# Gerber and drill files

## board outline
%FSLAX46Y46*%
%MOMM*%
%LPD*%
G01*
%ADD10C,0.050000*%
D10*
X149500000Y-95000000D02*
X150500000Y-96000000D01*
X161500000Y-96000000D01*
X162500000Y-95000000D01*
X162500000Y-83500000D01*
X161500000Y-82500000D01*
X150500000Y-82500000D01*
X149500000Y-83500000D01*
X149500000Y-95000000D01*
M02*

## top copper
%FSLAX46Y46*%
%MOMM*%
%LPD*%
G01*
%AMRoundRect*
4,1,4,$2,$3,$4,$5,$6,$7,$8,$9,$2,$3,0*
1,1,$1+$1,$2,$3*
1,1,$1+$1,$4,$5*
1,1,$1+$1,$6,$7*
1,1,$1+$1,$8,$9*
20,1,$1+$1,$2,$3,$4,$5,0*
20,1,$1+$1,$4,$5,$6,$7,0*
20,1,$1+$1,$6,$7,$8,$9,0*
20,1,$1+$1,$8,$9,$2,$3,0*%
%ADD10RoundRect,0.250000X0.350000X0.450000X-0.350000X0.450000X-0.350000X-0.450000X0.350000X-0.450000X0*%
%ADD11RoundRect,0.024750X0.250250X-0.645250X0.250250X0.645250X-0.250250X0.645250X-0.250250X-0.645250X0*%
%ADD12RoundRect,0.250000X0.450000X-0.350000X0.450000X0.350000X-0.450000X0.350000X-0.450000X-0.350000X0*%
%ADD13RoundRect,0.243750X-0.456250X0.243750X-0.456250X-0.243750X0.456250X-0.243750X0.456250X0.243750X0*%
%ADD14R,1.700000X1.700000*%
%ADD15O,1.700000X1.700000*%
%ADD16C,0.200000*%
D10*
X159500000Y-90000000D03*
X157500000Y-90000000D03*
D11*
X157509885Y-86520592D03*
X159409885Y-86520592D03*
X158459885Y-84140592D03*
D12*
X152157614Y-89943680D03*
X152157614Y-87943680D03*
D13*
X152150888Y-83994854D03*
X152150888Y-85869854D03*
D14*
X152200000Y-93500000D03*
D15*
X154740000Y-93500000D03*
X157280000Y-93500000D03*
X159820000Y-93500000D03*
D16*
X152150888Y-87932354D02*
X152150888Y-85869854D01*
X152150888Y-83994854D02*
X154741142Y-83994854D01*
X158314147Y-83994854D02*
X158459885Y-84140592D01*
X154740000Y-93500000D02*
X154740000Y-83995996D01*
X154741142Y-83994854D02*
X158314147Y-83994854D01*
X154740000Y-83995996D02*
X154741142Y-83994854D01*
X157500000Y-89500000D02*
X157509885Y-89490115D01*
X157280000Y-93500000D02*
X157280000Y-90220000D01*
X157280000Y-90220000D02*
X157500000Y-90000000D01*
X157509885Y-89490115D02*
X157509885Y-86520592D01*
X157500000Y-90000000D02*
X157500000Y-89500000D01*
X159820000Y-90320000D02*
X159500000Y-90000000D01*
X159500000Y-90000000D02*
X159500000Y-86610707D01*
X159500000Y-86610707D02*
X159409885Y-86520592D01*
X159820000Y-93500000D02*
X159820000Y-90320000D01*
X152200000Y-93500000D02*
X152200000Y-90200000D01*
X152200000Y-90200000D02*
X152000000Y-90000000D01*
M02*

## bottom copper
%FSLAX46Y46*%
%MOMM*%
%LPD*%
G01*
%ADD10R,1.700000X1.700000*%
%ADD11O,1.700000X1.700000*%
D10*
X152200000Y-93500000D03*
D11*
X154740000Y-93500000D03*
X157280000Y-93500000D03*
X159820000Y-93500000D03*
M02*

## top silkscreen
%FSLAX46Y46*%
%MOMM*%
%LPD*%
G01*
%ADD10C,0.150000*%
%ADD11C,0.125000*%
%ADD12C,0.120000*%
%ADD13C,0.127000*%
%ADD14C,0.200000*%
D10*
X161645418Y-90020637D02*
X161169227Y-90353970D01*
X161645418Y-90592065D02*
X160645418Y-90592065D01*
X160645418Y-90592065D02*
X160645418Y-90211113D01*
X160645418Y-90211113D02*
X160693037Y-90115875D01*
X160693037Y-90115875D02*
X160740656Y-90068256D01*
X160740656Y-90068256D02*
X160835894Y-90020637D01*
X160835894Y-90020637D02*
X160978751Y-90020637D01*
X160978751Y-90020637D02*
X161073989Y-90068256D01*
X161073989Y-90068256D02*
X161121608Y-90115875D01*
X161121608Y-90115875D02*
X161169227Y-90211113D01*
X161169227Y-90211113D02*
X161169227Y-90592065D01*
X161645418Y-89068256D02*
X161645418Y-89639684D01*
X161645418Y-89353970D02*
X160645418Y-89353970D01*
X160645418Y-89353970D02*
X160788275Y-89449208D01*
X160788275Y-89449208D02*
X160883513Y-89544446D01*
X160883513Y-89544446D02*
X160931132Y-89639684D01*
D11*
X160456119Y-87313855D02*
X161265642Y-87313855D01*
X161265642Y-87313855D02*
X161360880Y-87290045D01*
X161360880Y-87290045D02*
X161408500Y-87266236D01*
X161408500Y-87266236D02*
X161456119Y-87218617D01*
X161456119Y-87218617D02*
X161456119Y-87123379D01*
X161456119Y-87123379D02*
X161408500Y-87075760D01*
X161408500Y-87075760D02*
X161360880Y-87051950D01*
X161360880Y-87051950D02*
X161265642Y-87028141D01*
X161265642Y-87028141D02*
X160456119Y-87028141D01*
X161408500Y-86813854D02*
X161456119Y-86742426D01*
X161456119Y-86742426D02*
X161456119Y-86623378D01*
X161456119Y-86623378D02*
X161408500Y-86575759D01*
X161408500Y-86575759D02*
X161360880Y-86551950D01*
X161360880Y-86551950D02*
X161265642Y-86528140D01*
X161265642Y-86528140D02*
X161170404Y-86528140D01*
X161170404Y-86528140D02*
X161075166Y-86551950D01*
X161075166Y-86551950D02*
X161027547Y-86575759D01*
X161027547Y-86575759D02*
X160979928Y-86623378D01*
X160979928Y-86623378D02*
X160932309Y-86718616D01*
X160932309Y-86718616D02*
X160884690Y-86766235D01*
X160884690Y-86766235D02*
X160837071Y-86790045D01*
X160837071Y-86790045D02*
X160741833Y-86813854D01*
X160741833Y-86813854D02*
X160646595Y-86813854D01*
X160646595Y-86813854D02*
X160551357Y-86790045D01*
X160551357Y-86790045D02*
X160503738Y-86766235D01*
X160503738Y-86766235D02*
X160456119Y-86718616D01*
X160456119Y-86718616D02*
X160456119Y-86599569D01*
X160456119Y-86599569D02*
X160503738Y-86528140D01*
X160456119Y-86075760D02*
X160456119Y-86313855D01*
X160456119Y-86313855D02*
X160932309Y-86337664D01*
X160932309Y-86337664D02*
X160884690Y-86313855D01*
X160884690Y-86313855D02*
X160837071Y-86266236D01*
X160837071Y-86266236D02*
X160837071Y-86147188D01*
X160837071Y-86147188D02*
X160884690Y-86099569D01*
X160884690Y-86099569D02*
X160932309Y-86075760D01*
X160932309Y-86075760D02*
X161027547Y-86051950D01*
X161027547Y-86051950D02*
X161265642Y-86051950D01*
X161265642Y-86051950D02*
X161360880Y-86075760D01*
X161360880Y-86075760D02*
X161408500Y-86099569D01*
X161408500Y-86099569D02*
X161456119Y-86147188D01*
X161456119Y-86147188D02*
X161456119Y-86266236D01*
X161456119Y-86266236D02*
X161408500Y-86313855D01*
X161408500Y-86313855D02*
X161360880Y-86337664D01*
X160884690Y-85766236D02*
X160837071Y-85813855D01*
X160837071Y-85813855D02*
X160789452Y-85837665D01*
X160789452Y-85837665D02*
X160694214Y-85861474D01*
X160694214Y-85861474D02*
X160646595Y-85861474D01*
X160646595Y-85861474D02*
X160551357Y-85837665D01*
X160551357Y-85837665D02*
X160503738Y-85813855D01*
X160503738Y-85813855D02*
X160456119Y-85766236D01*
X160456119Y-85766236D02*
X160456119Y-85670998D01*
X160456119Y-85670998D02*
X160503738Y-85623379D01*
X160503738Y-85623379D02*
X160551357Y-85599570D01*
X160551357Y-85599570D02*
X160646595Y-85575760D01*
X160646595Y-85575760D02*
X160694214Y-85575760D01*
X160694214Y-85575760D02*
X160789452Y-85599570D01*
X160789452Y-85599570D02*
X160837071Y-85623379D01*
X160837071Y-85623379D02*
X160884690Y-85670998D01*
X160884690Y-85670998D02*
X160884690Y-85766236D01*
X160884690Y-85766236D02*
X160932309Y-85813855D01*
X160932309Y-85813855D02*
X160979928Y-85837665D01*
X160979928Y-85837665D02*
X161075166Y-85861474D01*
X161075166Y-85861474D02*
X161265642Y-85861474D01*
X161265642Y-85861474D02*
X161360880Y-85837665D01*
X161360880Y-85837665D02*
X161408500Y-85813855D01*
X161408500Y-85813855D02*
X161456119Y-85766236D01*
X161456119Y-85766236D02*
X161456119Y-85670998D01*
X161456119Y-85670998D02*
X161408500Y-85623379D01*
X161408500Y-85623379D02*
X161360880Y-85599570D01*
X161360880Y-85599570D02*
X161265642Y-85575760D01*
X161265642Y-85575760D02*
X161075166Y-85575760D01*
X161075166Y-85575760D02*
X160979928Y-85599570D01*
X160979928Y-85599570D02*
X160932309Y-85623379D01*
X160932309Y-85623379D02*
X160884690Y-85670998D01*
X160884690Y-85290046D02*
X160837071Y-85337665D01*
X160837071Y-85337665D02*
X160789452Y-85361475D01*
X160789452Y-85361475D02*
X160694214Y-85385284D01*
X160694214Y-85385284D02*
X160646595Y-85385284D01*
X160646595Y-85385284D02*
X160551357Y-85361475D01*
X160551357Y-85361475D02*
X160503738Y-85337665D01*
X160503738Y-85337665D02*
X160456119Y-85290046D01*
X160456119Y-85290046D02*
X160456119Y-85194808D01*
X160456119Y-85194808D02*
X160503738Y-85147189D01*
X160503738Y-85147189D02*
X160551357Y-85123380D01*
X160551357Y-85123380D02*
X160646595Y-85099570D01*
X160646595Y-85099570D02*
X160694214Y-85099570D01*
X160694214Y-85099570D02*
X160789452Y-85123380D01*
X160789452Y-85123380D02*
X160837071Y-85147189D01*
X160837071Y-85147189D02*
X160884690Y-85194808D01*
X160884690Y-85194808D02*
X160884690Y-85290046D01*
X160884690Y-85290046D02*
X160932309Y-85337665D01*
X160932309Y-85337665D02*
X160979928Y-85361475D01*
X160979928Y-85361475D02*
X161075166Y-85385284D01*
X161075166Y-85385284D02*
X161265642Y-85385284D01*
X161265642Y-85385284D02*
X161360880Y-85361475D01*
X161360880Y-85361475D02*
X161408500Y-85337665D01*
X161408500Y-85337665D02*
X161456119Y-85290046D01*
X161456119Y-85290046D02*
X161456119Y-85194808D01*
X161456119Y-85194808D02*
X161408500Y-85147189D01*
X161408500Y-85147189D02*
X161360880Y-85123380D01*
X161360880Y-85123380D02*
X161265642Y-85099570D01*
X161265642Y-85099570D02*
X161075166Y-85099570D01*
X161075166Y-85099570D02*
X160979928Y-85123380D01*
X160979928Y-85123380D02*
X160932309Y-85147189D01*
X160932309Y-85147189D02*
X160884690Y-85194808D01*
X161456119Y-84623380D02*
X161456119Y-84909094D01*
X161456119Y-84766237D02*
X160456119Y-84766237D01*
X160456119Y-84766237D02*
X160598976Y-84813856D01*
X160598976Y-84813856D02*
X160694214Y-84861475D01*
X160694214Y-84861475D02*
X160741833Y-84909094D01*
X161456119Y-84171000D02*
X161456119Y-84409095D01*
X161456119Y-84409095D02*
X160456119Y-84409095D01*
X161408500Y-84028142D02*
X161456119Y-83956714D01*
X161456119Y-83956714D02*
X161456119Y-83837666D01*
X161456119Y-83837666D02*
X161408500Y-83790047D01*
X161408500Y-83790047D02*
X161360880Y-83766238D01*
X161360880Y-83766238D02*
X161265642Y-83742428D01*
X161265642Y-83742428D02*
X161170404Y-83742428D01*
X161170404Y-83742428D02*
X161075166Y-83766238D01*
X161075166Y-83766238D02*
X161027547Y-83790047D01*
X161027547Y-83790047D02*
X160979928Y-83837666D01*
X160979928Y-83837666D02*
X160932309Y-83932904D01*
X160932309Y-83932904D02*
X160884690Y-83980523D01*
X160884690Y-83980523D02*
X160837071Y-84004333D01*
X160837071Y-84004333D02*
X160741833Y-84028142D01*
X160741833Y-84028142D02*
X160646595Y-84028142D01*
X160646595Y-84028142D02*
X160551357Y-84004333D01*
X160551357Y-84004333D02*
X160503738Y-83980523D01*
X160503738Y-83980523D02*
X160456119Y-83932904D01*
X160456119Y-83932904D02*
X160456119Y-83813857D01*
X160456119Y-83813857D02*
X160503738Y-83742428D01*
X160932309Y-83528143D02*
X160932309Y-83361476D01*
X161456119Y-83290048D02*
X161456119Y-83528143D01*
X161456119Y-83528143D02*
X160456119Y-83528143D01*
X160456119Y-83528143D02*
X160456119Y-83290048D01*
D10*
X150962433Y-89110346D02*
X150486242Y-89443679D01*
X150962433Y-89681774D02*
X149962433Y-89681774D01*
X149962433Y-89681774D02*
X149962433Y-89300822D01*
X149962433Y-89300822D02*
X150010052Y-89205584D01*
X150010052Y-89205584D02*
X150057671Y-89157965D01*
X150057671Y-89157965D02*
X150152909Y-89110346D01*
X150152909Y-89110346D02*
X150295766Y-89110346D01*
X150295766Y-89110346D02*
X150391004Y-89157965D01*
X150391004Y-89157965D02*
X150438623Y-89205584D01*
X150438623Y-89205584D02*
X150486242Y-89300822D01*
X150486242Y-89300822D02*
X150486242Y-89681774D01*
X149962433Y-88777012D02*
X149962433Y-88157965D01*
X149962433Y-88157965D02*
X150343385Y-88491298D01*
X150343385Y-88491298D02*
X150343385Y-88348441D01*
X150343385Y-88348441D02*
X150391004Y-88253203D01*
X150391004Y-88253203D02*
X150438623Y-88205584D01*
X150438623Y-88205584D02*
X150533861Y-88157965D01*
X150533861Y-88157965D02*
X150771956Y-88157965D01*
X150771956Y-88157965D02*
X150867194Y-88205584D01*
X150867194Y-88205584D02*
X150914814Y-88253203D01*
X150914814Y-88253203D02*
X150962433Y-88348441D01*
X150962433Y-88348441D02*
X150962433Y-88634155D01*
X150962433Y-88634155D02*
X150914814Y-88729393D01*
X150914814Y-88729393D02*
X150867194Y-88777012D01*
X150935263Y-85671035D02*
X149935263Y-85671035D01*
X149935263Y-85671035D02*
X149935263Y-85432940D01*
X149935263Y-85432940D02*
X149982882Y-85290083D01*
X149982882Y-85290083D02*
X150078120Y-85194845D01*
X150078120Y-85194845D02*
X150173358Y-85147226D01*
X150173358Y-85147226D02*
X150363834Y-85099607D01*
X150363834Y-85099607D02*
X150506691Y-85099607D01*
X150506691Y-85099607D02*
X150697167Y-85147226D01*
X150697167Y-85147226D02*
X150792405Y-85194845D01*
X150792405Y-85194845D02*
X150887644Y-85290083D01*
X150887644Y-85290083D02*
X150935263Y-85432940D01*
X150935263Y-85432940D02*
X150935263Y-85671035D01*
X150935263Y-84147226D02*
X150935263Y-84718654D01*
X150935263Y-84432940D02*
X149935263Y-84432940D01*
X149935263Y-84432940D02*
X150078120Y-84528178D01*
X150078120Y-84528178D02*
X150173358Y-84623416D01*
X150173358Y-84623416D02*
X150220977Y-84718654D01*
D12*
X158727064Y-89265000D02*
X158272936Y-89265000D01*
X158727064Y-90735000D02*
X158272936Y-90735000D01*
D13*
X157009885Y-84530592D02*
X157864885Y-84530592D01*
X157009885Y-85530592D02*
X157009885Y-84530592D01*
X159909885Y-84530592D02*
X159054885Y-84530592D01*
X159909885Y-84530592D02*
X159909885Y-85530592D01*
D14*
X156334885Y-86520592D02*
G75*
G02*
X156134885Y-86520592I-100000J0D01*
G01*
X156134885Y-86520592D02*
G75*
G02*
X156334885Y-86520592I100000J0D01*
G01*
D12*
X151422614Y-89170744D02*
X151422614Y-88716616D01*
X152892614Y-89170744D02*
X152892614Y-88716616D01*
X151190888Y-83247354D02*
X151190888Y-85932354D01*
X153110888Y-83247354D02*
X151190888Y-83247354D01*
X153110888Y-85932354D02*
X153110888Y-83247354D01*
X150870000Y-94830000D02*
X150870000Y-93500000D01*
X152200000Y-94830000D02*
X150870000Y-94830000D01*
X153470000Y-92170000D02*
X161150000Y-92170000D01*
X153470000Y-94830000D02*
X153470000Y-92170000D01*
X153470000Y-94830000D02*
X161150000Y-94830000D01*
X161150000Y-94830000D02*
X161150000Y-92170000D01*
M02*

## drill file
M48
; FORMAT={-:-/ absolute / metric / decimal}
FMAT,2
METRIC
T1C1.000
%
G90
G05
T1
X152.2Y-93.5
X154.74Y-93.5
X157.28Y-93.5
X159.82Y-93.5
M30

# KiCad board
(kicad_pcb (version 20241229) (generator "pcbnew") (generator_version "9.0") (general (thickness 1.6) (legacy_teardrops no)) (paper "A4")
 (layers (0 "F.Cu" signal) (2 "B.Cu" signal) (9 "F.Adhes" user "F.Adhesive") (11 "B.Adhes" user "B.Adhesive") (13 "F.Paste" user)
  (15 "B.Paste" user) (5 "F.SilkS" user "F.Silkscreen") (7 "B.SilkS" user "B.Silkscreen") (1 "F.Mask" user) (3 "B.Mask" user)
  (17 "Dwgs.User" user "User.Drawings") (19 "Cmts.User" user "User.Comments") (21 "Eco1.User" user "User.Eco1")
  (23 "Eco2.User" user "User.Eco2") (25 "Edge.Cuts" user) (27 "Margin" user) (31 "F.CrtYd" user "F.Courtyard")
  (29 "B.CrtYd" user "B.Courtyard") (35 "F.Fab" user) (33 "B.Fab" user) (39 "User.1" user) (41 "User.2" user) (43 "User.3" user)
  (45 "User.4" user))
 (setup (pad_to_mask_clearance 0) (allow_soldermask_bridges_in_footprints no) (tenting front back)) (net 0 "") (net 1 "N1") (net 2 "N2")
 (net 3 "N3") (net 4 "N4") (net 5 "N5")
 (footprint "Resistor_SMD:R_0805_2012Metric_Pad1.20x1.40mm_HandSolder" (layer "F.Cu") (at 158.5 90 180)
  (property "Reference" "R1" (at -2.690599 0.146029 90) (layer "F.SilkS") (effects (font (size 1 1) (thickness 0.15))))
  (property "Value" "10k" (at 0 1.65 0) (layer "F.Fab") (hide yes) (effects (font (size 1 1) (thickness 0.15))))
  (fp_line (start -0.227064 0.735) (end 0.227064 0.735) (stroke (width 0.12) (type solid)) (layer "F.SilkS"))
  (fp_line (start -0.227064 -0.735) (end 0.227064 -0.735) (stroke (width 0.12) (type solid)) (layer "F.SilkS"))
  (pad "1" smd roundrect (at -1 0 180) (size 1.2 1.4) (layers "F.Cu" "F.Mask" "F.Paste") (roundrect_rratio 0.208333) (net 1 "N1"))
  (pad "2" smd roundrect (at 1 0 180) (size 1.2 1.4) (layers "F.Cu" "F.Mask" "F.Paste") (roundrect_rratio 0.208333) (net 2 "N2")))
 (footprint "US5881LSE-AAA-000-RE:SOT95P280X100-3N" (layer "F.Cu") (at 158.459885 85.330592 90)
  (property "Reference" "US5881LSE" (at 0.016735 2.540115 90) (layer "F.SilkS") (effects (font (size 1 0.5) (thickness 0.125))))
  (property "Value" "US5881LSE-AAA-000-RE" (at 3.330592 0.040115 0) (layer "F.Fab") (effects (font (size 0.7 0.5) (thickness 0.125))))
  (fp_line (start 0.8 -1.45) (end 0.8 -0.595) (stroke (width 0.127) (type solid)) (layer "F.SilkS"))
  (fp_line (start -0.2 -1.45) (end 0.8 -1.45) (stroke (width 0.127) (type solid)) (layer "F.SilkS"))
  (fp_line (start 0.8 1.45) (end 0.8 0.595) (stroke (width 0.127) (type solid)) (layer "F.SilkS"))
  (fp_line (start 0.8 1.45) (end -0.2 1.45) (stroke (width 0.127) (type solid)) (layer "F.SilkS"))
  (fp_circle (center -1.19 -2.225) (end -1.09 -2.225) (stroke (width 0.2) (type solid)) (fill no) (layer "F.SilkS"))
  (pad "1" smd roundrect (at -1.19 -0.95 90) (size 1.34 0.55) (layers "F.Cu" "F.Mask" "F.Paste") (roundrect_rratio 0.045) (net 2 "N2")
   (solder_mask_margin 0.102))
  (pad "2" smd roundrect (at -1.19 0.95 90) (size 1.34 0.55) (layers "F.Cu" "F.Mask" "F.Paste") (roundrect_rratio 0.045) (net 1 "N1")
   (solder_mask_margin 0.102))
  (pad "3" smd roundrect (at 1.19 0 90) (size 1.34 0.55) (layers "F.Cu" "F.Mask" "F.Paste") (roundrect_rratio 0.045) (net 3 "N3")
   (solder_mask_margin 0.102)))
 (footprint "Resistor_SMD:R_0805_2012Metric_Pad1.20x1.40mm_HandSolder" (layer "F.Cu") (at 152.157614 88.94368 90)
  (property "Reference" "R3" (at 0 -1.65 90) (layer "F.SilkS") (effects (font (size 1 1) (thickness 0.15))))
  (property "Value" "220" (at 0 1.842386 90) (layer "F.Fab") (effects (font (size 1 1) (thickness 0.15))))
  (fp_line (start -0.227064 -0.735) (end 0.227064 -0.735) (stroke (width 0.12) (type solid)) (layer "F.SilkS"))
  (fp_line (start -0.227064 0.735) (end 0.227064 0.735) (stroke (width 0.12) (type solid)) (layer "F.SilkS"))
  (pad "1" smd roundrect (at -1 0 90) (size 1.2 1.4) (layers "F.Cu" "F.Mask" "F.Paste") (roundrect_rratio 0.208333) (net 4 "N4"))
  (pad "2" smd roundrect (at 1 0 90) (size 1.2 1.4) (layers "F.Cu" "F.Mask" "F.Paste") (roundrect_rratio 0.208333) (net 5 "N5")))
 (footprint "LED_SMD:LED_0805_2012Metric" (layer "F.Cu") (at 152.150888 84.932354 -90)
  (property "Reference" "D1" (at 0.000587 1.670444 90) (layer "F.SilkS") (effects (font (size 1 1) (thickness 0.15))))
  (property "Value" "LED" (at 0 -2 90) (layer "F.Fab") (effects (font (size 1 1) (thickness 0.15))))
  (fp_line (start -1.685 0.96) (end 1 0.96) (stroke (width 0.12) (type solid)) (layer "F.SilkS"))
  (fp_line (start -1.685 -0.96) (end -1.685 0.96) (stroke (width 0.12) (type solid)) (layer "F.SilkS"))
  (fp_line (start 1 -0.96) (end -1.685 -0.96) (stroke (width 0.12) (type solid)) (layer "F.SilkS"))
  (pad "1" smd roundrect (at -0.9375 0 270) (size 0.975 1.4) (layers "F.Cu" "F.Mask" "F.Paste") (roundrect_rratio 0.25) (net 3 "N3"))
  (pad "2" smd roundrect (at 0.9375 0 270) (size 0.975 1.4) (layers "F.Cu" "F.Mask" "F.Paste") (roundrect_rratio 0.25) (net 5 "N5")))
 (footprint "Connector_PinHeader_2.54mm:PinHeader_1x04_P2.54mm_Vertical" (layer "F.Cu") (at 152.2 93.5 90)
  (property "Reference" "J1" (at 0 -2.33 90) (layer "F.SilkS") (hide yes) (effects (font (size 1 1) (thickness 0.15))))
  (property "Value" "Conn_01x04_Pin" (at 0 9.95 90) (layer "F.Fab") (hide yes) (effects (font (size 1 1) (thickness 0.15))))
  (fp_line (start -1.33 -1.33) (end 0 -1.33) (stroke (width 0.12) (type solid)) (layer "F.SilkS"))
  (fp_line (start -1.33 0) (end -1.33 -1.33) (stroke (width 0.12) (type solid)) (layer "F.SilkS"))
  (fp_line (start 1.33 1.27) (end 1.33 8.95) (stroke (width 0.12) (type solid)) (layer "F.SilkS"))
  (fp_line (start -1.33 1.27) (end 1.33 1.27) (stroke (width 0.12) (type solid)) (layer "F.SilkS"))
  (fp_line (start -1.33 1.27) (end -1.33 8.95) (stroke (width 0.12) (type solid)) (layer "F.SilkS"))
  (fp_line (start -1.33 8.95) (end 1.33 8.95) (stroke (width 0.12) (type solid)) (layer "F.SilkS"))
  (pad "1" thru_hole rect (at 0 0 90) (size 1.7 1.7) (drill 1) (layers "*.Cu" "*.Mask") (remove_unused_layers no) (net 4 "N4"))
  (pad "2" thru_hole oval (at 0 2.54 90) (size 1.7 1.7) (drill 1) (layers "*.Cu" "*.Mask") (remove_unused_layers no) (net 3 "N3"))
  (pad "3" thru_hole oval (at 0 5.08 90) (size 1.7 1.7) (drill 1) (layers "*.Cu" "*.Mask") (remove_unused_layers no) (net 2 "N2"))
  (pad "4" thru_hole oval (at 0 7.62 90) (size 1.7 1.7) (drill 1) (layers "*.Cu" "*.Mask") (remove_unused_layers no) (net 1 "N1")))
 (gr_poly
  (pts (xy 149.5 95) (xy 150.5 96) (xy 161.5 96) (xy 162.5 95) (xy 162.5 83.5) (xy 161.5 82.5) (xy 150.5 82.5) (xy 149.5 83.5))
  (stroke (width 0.05) (type solid)) (fill no) (layer "Edge.Cuts"))
 (segment (start 152.150888 87.932354) (end 152.150888 85.869854) (width 0.2) (layer "F.Cu") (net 5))
 (segment (start 152.150888 83.994854) (end 154.741142 83.994854) (width 0.2) (layer "F.Cu") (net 3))
 (segment (start 158.314147 83.994854) (end 158.459885 84.140592) (width 0.2) (layer "F.Cu") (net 3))
 (segment (start 154.74 93.5) (end 154.74 83.995996) (width 0.2) (layer "F.Cu") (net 3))
 (segment (start 154.741142 83.994854) (end 158.314147 83.994854) (width 0.2) (layer "F.Cu") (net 3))
 (segment (start 154.74 83.995996) (end 154.741142 83.994854) (width 0.2) (layer "F.Cu") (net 3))
 (segment (start 157.5 89.5) (end 157.509885 89.490115) (width 0.2) (layer "F.Cu") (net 2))
 (segment (start 157.28 93.5) (end 157.28 90.22) (width 0.2) (layer "F.Cu") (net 2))
 (segment (start 157.28 90.22) (end 157.5 90) (width 0.2) (layer "F.Cu") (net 2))
 (segment (start 157.509885 89.490115) (end 157.509885 86.520592) (width 0.2) (layer "F.Cu") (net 2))
 (segment (start 157.5 90) (end 157.5 89.5) (width 0.2) (layer "F.Cu") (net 2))
 (segment (start 159.82 90.32) (end 159.5 90) (width 0.2) (layer "F.Cu") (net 1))
 (segment (start 159.5 90) (end 159.5 86.610707) (width 0.2) (layer "F.Cu") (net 1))
 (segment (start 159.5 86.610707) (end 159.409885 86.520592) (width 0.2) (layer "F.Cu") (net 1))
 (segment (start 159.82 93.5) (end 159.82 90.32) (width 0.2) (layer "F.Cu") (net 1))
 (segment (start 152.2 93.5) (end 152.2 90.2) (width 0.2) (layer "F.Cu") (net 4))
 (segment (start 152.2 90.2) (end 152 90) (width 0.2) (layer "F.Cu") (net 4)))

